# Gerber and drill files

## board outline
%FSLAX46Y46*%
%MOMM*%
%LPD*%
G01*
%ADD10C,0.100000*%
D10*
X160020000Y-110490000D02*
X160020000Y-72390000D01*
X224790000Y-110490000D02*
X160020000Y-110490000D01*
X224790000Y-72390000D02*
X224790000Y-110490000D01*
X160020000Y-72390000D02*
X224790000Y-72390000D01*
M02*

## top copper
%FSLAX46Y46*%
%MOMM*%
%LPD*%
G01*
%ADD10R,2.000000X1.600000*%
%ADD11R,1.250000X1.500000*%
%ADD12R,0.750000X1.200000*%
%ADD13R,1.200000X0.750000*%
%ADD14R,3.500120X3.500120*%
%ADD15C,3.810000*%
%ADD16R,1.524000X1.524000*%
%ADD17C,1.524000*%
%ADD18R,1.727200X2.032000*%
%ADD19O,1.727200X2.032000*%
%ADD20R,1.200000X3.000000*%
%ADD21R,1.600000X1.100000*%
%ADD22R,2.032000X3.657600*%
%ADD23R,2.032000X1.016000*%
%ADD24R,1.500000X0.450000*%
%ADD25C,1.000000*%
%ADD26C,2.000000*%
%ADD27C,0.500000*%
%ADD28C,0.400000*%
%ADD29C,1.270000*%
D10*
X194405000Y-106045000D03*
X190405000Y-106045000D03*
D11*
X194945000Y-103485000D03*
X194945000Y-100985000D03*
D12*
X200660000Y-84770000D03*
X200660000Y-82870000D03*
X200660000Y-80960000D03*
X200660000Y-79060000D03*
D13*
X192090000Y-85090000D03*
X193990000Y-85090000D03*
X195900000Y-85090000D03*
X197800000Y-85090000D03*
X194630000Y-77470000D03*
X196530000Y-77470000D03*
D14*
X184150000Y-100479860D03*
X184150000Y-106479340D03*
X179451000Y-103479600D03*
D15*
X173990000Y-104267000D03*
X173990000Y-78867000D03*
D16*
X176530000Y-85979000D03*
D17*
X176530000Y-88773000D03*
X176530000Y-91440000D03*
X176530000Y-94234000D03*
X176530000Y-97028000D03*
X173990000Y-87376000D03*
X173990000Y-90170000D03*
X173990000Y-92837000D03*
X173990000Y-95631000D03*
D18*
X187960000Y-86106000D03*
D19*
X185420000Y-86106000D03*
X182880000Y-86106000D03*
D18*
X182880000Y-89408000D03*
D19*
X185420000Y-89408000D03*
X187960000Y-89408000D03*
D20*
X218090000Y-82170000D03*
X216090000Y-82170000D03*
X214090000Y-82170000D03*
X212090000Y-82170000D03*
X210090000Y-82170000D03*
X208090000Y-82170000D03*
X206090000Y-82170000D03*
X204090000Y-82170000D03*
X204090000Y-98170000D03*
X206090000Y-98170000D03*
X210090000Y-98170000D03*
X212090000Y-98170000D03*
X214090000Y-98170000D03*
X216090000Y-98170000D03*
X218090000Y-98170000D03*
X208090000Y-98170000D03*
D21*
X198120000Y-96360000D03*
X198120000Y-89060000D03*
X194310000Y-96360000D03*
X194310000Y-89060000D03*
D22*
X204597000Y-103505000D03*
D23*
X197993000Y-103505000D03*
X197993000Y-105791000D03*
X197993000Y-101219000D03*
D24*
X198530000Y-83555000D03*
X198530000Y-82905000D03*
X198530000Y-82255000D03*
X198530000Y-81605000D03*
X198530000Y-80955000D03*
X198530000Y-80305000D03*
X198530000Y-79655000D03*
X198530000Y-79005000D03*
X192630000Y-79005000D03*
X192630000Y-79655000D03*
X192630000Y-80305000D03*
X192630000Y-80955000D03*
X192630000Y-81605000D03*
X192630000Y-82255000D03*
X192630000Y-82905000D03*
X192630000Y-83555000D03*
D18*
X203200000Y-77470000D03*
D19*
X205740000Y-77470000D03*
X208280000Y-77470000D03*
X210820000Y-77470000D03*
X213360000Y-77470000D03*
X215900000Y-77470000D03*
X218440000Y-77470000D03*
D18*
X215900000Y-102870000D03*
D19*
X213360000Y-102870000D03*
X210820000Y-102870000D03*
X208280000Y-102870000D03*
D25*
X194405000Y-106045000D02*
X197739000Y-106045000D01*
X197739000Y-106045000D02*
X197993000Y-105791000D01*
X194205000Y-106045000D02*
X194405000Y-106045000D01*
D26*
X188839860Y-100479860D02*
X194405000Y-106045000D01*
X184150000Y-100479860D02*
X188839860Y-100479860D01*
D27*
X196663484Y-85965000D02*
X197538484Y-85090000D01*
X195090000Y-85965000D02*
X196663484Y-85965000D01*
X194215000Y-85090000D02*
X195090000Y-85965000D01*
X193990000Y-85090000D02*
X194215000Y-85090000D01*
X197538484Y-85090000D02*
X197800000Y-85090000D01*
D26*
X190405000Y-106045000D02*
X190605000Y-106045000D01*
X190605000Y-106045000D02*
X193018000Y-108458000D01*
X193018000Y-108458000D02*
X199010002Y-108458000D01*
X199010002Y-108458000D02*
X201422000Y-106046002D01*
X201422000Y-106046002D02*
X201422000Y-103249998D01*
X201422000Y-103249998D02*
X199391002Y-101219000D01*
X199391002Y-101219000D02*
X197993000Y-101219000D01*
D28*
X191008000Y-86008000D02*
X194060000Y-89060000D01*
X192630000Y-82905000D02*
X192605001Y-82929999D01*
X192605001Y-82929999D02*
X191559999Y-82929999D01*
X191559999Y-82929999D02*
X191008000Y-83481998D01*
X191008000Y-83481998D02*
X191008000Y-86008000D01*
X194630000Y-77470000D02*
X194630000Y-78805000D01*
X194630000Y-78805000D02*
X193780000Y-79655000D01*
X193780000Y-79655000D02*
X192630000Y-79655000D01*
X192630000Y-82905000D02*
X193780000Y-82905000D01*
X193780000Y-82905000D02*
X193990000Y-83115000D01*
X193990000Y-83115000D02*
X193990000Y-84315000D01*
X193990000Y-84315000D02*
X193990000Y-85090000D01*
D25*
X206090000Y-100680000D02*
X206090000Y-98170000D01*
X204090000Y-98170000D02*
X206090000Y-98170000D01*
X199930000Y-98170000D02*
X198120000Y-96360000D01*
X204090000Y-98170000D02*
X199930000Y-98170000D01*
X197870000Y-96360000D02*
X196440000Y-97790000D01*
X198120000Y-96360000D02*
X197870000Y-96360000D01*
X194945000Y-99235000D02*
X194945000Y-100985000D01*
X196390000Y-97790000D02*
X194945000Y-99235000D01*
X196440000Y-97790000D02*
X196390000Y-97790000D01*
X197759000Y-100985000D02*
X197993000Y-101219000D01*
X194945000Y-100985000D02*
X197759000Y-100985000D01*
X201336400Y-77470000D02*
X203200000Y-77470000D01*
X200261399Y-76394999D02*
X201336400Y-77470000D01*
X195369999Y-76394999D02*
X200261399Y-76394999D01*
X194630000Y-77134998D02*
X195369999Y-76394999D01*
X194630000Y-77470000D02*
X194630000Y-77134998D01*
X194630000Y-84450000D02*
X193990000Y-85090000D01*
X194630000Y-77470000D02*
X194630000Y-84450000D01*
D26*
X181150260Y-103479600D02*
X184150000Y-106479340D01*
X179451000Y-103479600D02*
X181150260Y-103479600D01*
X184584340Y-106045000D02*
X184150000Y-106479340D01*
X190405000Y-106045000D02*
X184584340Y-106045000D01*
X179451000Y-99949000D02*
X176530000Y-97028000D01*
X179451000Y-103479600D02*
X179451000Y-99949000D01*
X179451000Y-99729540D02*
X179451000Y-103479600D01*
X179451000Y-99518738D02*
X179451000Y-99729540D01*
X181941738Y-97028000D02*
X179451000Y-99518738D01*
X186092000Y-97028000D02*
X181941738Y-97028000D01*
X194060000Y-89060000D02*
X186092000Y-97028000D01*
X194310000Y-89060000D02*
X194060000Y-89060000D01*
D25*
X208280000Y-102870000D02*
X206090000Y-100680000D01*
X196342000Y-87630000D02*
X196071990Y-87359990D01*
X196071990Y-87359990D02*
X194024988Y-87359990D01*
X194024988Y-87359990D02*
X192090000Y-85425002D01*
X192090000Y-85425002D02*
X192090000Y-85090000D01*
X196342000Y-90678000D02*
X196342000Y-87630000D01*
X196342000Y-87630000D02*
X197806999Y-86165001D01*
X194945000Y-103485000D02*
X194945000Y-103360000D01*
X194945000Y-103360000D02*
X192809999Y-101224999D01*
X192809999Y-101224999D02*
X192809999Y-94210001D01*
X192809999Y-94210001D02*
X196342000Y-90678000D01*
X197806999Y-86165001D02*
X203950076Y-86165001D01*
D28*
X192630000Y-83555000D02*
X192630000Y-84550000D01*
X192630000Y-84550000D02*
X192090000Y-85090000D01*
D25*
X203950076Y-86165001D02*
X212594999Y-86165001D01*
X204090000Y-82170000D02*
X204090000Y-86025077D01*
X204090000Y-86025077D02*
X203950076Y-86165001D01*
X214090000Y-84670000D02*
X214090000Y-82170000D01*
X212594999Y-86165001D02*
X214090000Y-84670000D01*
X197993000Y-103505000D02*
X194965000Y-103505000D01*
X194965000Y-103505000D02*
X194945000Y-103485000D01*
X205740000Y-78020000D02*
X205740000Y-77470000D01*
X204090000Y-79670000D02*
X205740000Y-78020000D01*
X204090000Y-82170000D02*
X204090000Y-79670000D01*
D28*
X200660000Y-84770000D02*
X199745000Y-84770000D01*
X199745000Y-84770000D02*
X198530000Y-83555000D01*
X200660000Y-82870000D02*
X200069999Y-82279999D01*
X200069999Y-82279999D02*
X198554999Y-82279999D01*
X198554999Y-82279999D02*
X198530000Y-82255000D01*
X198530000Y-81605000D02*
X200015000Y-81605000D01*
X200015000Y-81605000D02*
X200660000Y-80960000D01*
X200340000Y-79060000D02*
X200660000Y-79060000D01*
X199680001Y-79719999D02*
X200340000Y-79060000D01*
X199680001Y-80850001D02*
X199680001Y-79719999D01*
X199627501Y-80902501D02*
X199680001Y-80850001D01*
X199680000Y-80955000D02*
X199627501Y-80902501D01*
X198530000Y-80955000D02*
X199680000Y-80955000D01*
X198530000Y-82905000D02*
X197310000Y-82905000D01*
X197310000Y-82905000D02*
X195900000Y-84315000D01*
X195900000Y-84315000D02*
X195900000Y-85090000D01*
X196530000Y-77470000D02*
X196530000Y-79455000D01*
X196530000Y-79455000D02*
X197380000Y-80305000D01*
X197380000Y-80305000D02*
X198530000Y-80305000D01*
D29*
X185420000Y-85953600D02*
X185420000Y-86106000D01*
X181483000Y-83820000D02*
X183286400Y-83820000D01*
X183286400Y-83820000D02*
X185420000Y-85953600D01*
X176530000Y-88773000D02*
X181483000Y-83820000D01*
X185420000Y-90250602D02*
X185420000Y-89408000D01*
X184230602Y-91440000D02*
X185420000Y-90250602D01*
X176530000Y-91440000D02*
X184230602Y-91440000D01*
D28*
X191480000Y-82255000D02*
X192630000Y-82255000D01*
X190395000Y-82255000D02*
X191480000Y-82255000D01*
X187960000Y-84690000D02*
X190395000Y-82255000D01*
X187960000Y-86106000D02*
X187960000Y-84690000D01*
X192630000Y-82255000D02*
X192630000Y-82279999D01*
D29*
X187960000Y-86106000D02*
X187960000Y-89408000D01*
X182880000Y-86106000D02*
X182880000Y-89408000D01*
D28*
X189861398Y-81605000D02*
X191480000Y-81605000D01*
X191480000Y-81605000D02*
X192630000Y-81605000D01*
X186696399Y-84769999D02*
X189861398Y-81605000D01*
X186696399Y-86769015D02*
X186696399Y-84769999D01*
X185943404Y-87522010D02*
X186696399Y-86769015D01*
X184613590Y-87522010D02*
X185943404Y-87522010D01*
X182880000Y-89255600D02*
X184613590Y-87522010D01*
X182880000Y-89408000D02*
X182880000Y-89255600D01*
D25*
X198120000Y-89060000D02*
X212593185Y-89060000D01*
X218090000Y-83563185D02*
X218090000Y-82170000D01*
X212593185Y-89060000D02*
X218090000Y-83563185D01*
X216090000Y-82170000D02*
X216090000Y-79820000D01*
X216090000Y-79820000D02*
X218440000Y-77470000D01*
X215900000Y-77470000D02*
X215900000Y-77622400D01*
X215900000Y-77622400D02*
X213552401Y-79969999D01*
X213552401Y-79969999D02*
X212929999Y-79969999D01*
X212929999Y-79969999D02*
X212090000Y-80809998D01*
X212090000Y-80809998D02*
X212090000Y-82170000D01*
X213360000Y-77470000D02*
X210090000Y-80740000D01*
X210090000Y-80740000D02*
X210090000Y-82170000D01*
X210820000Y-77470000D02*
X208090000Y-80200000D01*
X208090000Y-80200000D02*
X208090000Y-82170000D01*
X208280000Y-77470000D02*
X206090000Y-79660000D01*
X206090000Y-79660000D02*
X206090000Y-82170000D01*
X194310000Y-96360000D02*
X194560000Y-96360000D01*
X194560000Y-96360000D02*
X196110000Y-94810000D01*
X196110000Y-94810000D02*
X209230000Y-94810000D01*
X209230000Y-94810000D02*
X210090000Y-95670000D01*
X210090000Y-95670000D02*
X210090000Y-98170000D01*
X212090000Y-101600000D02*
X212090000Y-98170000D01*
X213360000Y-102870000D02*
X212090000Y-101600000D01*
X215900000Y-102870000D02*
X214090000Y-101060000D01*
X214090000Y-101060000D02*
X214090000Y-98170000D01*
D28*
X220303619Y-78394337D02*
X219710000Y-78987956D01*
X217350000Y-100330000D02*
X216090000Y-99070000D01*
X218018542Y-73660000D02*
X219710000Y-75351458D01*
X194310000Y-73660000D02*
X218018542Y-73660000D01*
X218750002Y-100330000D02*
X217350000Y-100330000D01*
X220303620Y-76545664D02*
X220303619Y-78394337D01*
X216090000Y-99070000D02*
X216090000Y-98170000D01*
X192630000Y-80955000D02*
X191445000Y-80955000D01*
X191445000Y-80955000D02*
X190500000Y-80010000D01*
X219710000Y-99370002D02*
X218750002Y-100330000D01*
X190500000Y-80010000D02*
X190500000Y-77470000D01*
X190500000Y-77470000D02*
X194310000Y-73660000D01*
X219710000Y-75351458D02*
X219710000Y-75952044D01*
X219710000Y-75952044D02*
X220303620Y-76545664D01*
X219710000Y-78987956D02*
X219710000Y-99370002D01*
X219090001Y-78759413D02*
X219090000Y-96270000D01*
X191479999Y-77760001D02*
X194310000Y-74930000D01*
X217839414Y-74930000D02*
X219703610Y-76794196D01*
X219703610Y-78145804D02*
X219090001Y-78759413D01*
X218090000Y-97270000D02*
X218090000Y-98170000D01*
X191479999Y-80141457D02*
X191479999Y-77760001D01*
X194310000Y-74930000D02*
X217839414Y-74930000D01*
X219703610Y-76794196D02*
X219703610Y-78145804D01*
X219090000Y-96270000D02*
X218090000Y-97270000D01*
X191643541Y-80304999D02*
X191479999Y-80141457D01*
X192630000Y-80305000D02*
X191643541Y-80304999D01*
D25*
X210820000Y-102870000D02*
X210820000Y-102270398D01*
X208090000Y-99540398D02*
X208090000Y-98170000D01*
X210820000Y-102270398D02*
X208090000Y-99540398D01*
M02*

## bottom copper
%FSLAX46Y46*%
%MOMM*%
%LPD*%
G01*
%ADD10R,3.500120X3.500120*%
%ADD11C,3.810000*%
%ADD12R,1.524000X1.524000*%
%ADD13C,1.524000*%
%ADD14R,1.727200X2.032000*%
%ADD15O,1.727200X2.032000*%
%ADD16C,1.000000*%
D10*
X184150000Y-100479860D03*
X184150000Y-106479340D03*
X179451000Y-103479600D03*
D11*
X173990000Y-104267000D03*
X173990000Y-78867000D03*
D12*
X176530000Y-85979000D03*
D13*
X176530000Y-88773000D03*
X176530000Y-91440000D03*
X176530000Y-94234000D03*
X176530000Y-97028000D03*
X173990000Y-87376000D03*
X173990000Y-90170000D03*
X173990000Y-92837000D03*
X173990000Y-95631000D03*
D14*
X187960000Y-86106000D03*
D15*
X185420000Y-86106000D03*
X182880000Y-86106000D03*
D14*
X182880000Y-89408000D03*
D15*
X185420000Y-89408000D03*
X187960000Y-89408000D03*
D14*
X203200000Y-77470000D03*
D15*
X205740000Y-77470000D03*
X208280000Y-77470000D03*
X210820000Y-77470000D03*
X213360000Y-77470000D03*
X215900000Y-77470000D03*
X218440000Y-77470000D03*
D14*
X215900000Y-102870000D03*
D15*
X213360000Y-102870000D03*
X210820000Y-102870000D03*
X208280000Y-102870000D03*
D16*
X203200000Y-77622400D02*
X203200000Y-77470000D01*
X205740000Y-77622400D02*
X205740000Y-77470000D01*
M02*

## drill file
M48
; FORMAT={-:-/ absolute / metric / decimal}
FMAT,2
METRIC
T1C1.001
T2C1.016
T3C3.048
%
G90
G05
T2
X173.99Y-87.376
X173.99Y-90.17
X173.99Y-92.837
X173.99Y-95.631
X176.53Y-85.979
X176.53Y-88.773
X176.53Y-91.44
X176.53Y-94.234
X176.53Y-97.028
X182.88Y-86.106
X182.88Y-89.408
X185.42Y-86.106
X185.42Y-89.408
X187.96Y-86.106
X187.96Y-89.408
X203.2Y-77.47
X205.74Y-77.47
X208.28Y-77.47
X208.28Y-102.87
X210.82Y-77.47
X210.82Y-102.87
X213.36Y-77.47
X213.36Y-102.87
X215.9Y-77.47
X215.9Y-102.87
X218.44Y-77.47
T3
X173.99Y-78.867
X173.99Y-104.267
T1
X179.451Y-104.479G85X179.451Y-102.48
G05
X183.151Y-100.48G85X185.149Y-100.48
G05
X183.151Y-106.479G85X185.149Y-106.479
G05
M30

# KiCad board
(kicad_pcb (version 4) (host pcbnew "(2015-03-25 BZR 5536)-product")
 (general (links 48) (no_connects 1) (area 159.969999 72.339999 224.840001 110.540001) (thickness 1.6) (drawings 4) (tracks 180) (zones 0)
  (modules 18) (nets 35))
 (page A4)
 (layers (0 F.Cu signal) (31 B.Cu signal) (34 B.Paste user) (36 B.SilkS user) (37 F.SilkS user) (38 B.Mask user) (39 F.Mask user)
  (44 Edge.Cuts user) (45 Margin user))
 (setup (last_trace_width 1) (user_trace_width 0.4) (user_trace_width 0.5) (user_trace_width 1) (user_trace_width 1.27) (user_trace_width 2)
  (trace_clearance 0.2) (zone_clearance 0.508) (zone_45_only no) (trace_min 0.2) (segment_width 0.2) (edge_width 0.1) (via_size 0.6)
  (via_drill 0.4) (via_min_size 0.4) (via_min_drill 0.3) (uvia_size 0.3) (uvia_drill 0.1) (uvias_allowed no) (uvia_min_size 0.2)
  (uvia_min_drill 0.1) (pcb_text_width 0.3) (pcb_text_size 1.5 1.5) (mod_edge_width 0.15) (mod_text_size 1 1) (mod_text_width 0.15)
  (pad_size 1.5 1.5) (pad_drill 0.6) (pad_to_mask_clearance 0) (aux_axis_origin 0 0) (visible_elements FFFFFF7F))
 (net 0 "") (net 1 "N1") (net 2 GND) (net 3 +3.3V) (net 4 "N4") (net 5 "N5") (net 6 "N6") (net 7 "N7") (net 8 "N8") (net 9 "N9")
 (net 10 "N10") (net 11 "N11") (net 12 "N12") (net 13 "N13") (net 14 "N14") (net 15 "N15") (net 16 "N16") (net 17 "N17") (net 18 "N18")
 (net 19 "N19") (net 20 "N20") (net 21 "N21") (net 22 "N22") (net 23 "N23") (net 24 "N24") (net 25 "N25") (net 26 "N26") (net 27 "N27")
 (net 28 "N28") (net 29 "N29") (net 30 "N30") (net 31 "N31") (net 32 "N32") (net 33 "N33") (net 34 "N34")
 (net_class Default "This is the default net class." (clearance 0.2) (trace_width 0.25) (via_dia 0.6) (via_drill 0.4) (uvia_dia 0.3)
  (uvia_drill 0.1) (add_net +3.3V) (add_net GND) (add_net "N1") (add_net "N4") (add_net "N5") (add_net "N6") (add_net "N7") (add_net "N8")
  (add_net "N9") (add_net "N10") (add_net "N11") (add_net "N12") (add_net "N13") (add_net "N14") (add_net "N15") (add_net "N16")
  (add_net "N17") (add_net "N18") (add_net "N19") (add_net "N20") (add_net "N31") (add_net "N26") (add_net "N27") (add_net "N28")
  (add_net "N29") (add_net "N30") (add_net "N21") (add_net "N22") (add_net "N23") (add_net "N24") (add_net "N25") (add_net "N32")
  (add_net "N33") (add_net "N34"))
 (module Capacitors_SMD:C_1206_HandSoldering (layer F.Cu) (at 192.405 106.045 180)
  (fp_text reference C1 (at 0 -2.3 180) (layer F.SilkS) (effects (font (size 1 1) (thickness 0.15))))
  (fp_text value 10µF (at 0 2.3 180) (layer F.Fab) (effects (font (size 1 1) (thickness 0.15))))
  (pad 1 smd rect (at -2 0 180) (size 2 1.6) (layers F.Cu F.Mask) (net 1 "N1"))
  (pad 2 smd rect (at 2 0 180) (size 2 1.6) (layers F.Cu F.Mask) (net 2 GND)))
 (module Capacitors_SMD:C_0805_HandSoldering (layer F.Cu) (at 194.945 102.235 90)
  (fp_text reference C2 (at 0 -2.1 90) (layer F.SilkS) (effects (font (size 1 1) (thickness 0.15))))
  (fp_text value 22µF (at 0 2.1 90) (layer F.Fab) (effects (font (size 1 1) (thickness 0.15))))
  (pad 1 smd rect (at -1.25 0 90) (size 1.5 1.25) (layers F.Cu F.Mask) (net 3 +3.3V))
  (pad 2 smd rect (at 1.25 0 90) (size 1.5 1.25) (layers F.Cu F.Mask) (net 2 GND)))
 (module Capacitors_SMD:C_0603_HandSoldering (layer F.Cu) (at 200.66 83.82 90)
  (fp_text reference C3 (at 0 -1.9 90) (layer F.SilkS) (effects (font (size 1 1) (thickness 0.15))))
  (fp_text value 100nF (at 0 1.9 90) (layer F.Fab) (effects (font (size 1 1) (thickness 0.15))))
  (pad 1 smd rect (at -0.95 0 90) (size 1.2 0.75) (layers F.Cu F.Mask) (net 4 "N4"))
  (pad 2 smd rect (at 0.95 0 90) (size 1.2 0.75) (layers F.Cu F.Mask) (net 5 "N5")))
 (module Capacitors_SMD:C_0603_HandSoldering (layer F.Cu) (at 200.66 80.01 90)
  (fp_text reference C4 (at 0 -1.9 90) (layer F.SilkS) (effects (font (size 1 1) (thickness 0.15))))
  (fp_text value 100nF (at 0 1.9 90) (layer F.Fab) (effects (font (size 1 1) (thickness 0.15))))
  (pad 1 smd rect (at -0.95 0 90) (size 1.2 0.75) (layers F.Cu F.Mask) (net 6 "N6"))
  (pad 2 smd rect (at 0.95 0 90) (size 1.2 0.75) (layers F.Cu F.Mask) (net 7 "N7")))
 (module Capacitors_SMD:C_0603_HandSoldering (layer F.Cu) (at 193.04 85.09)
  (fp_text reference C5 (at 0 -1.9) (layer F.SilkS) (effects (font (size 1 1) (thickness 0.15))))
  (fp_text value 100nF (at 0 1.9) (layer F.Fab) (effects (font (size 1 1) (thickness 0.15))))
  (pad 1 smd rect (at -0.95 0) (size 1.2 0.75) (layers F.Cu F.Mask) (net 3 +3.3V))
  (pad 2 smd rect (at 0.95 0) (size 1.2 0.75) (layers F.Cu F.Mask) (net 2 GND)))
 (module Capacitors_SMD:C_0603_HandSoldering (layer F.Cu) (at 196.85 85.09)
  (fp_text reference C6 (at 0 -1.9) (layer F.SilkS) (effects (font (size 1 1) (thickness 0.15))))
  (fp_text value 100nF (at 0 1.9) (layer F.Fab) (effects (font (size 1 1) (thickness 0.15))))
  (pad 1 smd rect (at -0.95 0) (size 1.2 0.75) (layers F.Cu F.Mask) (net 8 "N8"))
  (pad 2 smd rect (at 0.95 0) (size 1.2 0.75) (layers F.Cu F.Mask) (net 2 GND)))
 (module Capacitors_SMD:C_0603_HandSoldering (layer F.Cu) (at 195.58 77.47)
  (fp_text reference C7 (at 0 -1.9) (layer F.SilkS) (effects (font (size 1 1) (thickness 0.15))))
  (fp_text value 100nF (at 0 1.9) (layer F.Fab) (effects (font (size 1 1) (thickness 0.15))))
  (pad 1 smd rect (at -0.95 0) (size 1.2 0.75) (layers F.Cu F.Mask) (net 2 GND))
  (pad 2 smd rect (at 0.95 0) (size 1.2 0.75) (layers F.Cu F.Mask) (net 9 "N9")))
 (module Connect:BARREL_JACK (layer B.Cu) (at 184.15 106.68 90)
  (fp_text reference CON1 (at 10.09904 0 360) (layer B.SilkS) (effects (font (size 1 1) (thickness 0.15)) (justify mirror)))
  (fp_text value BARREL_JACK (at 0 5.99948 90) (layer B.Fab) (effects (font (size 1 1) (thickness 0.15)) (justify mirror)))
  (pad 1 thru_hole rect (at 6.20014 0 90) (size 3.50012 3.50012) (drill oval 1.00076 2.99974) (layers *.Cu *.Mask B.SilkS) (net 1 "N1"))
  (pad 2 thru_hole rect (at 0.20066 0 90) (size 3.50012 3.50012) (drill oval 1.00076 2.99974) (layers *.Cu *.Mask B.SilkS) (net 2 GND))
  (pad 3 thru_hole rect (at 3.2004 -4.699 90) (size 3.50012 3.50012) (drill oval 2.99974 1.00076) (layers *.Cu *.Mask B.SilkS) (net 2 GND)))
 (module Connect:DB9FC (layer B.Cu) (at 175.26 91.44 270)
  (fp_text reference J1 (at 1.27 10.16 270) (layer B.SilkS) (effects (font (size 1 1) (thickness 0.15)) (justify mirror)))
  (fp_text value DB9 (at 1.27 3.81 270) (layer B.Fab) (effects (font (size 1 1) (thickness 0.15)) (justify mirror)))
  (pad "" thru_hole circle (at 12.827 1.27 270) (size 3.81 3.81) (drill 3.048) (layers *.Cu *.Mask B.SilkS))
  (pad "" thru_hole circle (at -12.573 1.27 270) (size 3.81 3.81) (drill 3.048) (layers *.Cu *.Mask B.SilkS))
  (pad 1 thru_hole rect (at -5.461 -1.27 270) (size 1.524 1.524) (drill 1.016) (layers *.Cu *.Mask B.SilkS) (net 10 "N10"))
  (pad 2 thru_hole circle (at -2.667 -1.27 270) (size 1.524 1.524) (drill 1.016) (layers *.Cu *.Mask B.SilkS) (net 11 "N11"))
  (pad 3 thru_hole circle (at 0 -1.27 270) (size 1.524 1.524) (drill 1.016) (layers *.Cu *.Mask B.SilkS) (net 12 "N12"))
  (pad 4 thru_hole circle (at 2.794 -1.27 270) (size 1.524 1.524) (drill 1.016) (layers *.Cu *.Mask B.SilkS) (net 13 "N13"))
  (pad 5 thru_hole circle (at 5.588 -1.27 270) (size 1.524 1.524) (drill 1.016) (layers *.Cu *.Mask B.SilkS) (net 2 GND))
  (pad 6 thru_hole circle (at -4.064 1.27 270) (size 1.524 1.524) (drill 1.016) (layers *.Cu *.Mask B.SilkS) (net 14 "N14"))
  (pad 7 thru_hole circle (at -1.27 1.27 270) (size 1.524 1.524) (drill 1.016) (layers *.Cu *.Mask B.SilkS) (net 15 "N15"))
  (pad 8 thru_hole circle (at 1.397 1.27 270) (size 1.524 1.524) (drill 1.016) (layers *.Cu *.Mask B.SilkS) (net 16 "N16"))
  (pad 9 thru_hole circle (at 4.191 1.27 270) (size 1.524 1.524) (drill 1.016) (layers *.Cu *.Mask B.SilkS) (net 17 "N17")))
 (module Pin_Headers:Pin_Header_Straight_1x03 (layer B.Cu) (at 187.96 86.106 90)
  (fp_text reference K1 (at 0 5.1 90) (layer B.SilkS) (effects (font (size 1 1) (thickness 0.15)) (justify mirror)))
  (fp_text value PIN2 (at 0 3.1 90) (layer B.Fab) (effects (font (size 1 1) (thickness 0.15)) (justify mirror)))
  (pad 1 thru_hole rect (at 0 0 90) (size 2.032 1.7272) (drill 1.016) (layers *.Cu *.Mask B.SilkS) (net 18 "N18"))
  (pad 2 thru_hole oval (at 0 -2.54 90) (size 2.032 1.7272) (drill 1.016) (layers *.Cu *.Mask B.SilkS) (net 11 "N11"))
  (pad 3 thru_hole oval (at 0 -5.08 90) (size 2.032 1.7272) (drill 1.016) (layers *.Cu *.Mask B.SilkS) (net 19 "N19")))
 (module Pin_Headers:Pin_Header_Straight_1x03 (layer B.Cu) (at 182.88 89.408 270)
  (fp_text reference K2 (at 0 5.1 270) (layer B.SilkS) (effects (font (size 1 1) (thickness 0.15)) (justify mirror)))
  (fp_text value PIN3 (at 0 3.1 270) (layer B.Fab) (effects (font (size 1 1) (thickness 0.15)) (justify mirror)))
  (pad 1 thru_hole rect (at 0 0 270) (size 2.032 1.7272) (drill 1.016) (layers *.Cu *.Mask B.SilkS) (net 19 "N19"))
  (pad 2 thru_hole oval (at 0 -2.54 270) (size 2.032 1.7272) (drill 1.016) (layers *.Cu *.Mask B.SilkS) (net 12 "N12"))
  (pad 3 thru_hole oval (at 0 -5.08 270) (size 2.032 1.7272) (drill 1.016) (layers *.Cu *.Mask B.SilkS) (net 18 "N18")))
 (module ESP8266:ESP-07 (layer F.Cu) (at 212.09 90.17 180)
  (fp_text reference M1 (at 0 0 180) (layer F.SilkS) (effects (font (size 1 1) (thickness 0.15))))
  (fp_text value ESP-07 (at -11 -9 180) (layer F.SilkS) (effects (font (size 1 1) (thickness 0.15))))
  (pad 1 smd rect (at -6 8 180) (size 1.2 3) (layers F.Cu F.Mask) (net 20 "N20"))
  (pad 2 smd rect (at -4 8 180) (size 1.2 3) (layers F.Cu F.Mask) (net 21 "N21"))
  (pad 3 smd rect (at -2 8 180) (size 1.2 3) (layers F.Cu F.Mask) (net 3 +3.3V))
  (pad 4 smd rect (at 0 8 180) (size 1.2 3) (layers F.Cu F.Mask) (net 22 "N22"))
  (pad 5 smd rect (at 2 8 180) (size 1.2 3) (layers F.Cu F.Mask) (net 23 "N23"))
  (pad 6 smd rect (at 4 8 180) (size 1.2 3) (layers F.Cu F.Mask) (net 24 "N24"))
  (pad 7 smd rect (at 6 8 180) (size 1.2 3) (layers F.Cu F.Mask) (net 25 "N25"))
  (pad 8 smd rect (at 8 8 180) (size 1.2 3) (layers F.Cu F.Mask) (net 3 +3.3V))
  (pad 9 smd rect (at 8 -8 180) (size 1.2 3) (layers F.Cu F.Mask) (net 2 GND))
  (pad 10 smd rect (at 6 -8 180) (size 1.2 3) (layers F.Cu F.Mask) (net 2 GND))
  (pad 12 smd rect (at 2 -8 180) (size 1.2 3) (layers F.Cu F.Mask) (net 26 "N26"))
  (pad 13 smd rect (at 0 -8 180) (size 1.2 3) (layers F.Cu F.Mask) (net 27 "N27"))
  (pad 14 smd rect (at -2 -8 180) (size 1.2 3) (layers F.Cu F.Mask) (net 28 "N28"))
  (pad 15 smd rect (at -4 -8 180) (size 1.2 3) (layers F.Cu F.Mask) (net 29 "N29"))
  (pad 16 smd rect (at -6 -8 180) (size 1.2 3) (layers F.Cu F.Mask) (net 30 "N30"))
  (pad 11 smd rect (at 4 -8 180) (size 1.2 3) (layers F.Cu F.Mask) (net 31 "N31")))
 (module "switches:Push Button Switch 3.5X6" (layer F.Cu) (at 198.12 92.71 90)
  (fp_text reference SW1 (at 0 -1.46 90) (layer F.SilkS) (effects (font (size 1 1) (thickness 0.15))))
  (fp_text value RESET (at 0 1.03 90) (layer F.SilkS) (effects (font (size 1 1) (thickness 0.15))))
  (pad 1 smd rect (at -3.65 0 90) (size 1.1 1.6) (layers F.Cu F.Mask) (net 2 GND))
  (pad 2 smd rect (at 3.65 0 90) (size 1.1 1.6) (layers F.Cu F.Mask) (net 20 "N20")))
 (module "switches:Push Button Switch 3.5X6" (layer F.Cu) (at 194.31 92.71 90)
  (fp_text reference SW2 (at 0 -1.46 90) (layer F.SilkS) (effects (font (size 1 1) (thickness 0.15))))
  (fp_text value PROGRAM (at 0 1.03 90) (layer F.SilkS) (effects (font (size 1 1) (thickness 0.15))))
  (pad 1 smd rect (at -3.65 0 90) (size 1.1 1.6) (layers F.Cu F.Mask) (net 26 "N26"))
  (pad 2 smd rect (at 3.65 0 90) (size 1.1 1.6) (layers F.Cu F.Mask) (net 2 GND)))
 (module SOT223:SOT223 (layer F.Cu) (at 201.295 103.505 270)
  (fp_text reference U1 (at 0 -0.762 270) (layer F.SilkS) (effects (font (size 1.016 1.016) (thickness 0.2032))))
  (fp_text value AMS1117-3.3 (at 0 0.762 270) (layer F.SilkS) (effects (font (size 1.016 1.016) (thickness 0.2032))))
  (pad 4 smd rect (at 0 -3.302 270) (size 3.6576 2.032) (layers F.Cu F.Mask))
  (pad 2 smd rect (at 0 3.302 270) (size 1.016 2.032) (layers F.Cu F.Mask) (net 3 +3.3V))
  (pad 3 smd rect (at 2.286 3.302 270) (size 1.016 2.032) (layers F.Cu F.Mask) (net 1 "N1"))
  (pad 1 smd rect (at -2.286 3.302 270) (size 1.016 2.032) (layers F.Cu F.Mask) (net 2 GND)))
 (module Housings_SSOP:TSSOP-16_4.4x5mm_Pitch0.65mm (layer F.Cu) (at 195.58 81.28 180)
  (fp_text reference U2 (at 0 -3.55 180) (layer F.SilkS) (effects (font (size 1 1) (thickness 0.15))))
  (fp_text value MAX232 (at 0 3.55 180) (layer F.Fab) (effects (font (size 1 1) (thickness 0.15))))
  (pad 1 smd rect (at -2.95 -2.275 180) (size 1.5 0.45) (layers F.Cu F.Mask) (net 4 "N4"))
  (pad 2 smd rect (at -2.95 -1.625 180) (size 1.5 0.45) (layers F.Cu F.Mask) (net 8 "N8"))
  (pad 3 smd rect (at -2.95 -0.975 180) (size 1.5 0.45) (layers F.Cu F.Mask) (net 5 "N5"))
  (pad 4 smd rect (at -2.95 -0.325 180) (size 1.5 0.45) (layers F.Cu F.Mask) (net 6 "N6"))
  (pad 5 smd rect (at -2.95 0.325 180) (size 1.5 0.45) (layers F.Cu F.Mask) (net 7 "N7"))
  (pad 6 smd rect (at -2.95 0.975 180) (size 1.5 0.45) (layers F.Cu F.Mask) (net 9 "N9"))
  (pad 7 smd rect (at -2.95 1.625 180) (size 1.5 0.45) (layers F.Cu F.Mask) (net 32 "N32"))
  (pad 8 smd rect (at -2.95 2.275 180) (size 1.5 0.45) (layers F.Cu F.Mask) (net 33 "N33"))
  (pad 9 smd rect (at 2.95 2.275 180) (size 1.5 0.45) (layers F.Cu F.Mask) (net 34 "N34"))
  (pad 10 smd rect (at 2.95 1.625 180) (size 1.5 0.45) (layers F.Cu F.Mask) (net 2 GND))
  (pad 11 smd rect (at 2.95 0.975 180) (size 1.5 0.45) (layers F.Cu F.Mask) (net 30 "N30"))
  (pad 12 smd rect (at 2.95 0.325 180) (size 1.5 0.45) (layers F.Cu F.Mask) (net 29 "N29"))
  (pad 13 smd rect (at 2.95 -0.325 180) (size 1.5 0.45) (layers F.Cu F.Mask) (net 19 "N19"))
  (pad 14 smd rect (at 2.95 -0.975 180) (size 1.5 0.45) (layers F.Cu F.Mask) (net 18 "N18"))
  (pad 15 smd rect (at 2.95 -1.625 180) (size 1.5 0.45) (layers F.Cu F.Mask) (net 2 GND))
  (pad 16 smd rect (at 2.95 -2.275 180) (size 1.5 0.45) (layers F.Cu F.Mask) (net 3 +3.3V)))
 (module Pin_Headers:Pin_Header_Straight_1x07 (layer F.Cu) (at 203.2 77.47 90)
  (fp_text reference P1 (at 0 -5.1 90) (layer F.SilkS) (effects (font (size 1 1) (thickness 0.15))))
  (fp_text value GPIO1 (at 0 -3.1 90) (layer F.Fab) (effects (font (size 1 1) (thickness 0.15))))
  (pad 1 thru_hole rect (at 0 0 90) (size 2.032 1.7272) (drill 1.016) (layers *.Cu *.Mask F.SilkS) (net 2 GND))
  (pad 2 thru_hole oval (at 0 2.54 90) (size 2.032 1.7272) (drill 1.016) (layers *.Cu *.Mask F.SilkS) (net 3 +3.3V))
  (pad 3 thru_hole oval (at 0 5.08 90) (size 2.032 1.7272) (drill 1.016) (layers *.Cu *.Mask F.SilkS) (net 25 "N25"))
  (pad 4 thru_hole oval (at 0 7.62 90) (size 2.032 1.7272) (drill 1.016) (layers *.Cu *.Mask F.SilkS) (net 24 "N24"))
  (pad 5 thru_hole oval (at 0 10.16 90) (size 2.032 1.7272) (drill 1.016) (layers *.Cu *.Mask F.SilkS) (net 23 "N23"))
  (pad 6 thru_hole oval (at 0 12.7 90) (size 2.032 1.7272) (drill 1.016) (layers *.Cu *.Mask F.SilkS) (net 22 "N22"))
  (pad 7 thru_hole oval (at 0 15.24 90) (size 2.032 1.7272) (drill 1.016) (layers *.Cu *.Mask F.SilkS) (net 21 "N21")))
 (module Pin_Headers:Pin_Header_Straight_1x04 (layer F.Cu) (at 215.9 102.87 270)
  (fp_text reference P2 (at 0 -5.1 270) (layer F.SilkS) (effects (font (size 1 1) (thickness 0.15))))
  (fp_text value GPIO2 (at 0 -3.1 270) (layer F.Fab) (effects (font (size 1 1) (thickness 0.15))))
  (pad 1 thru_hole rect (at 0 0 270) (size 2.032 1.7272) (drill 1.016) (layers *.Cu *.Mask F.SilkS) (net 28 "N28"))
  (pad 2 thru_hole oval (at 0 2.54 270) (size 2.032 1.7272) (drill 1.016) (layers *.Cu *.Mask F.SilkS) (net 27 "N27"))
  (pad 3 thru_hole oval (at 0 5.08 270) (size 2.032 1.7272) (drill 1.016) (layers *.Cu *.Mask F.SilkS) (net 31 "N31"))
  (pad 4 thru_hole oval (at 0 7.62 270) (size 2.032 1.7272) (drill 1.016) (layers *.Cu *.Mask F.SilkS) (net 2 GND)))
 (gr_line (start 160.02 110.49) (end 160.02 72.39) (angle 90) (layer Edge.Cuts) (width 0.1))
 (gr_line (start 224.79 110.49) (end 160.02 110.49) (angle 90) (layer Edge.Cuts) (width 0.1))
 (gr_line (start 224.79 72.39) (end 224.79 110.49) (angle 90) (layer Edge.Cuts) (width 0.1))
 (gr_line (start 160.02 72.39) (end 224.79 72.39) (angle 90) (layer Edge.Cuts) (width 0.1))
 (segment (start 194.405 106.045) (end 197.739 106.045) (width 1) (layer F.Cu) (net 1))
 (segment (start 197.739 106.045) (end 197.993 105.791) (width 1) (layer F.Cu) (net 1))
 (segment (start 194.205 106.045) (end 194.405 106.045) (width 1) (layer F.Cu) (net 1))
 (segment (start 188.83986 100.47986) (end 194.405 106.045) (width 2) (layer F.Cu) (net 1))
 (segment (start 184.15 100.47986) (end 188.83986 100.47986) (width 2) (layer F.Cu) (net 1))
 (segment (start 196.663484 85.965) (end 197.538484 85.09) (width 0.5) (layer F.Cu) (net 2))
 (segment (start 195.09 85.965) (end 196.663484 85.965) (width 0.5) (layer F.Cu) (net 2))
 (segment (start 194.215 85.09) (end 195.09 85.965) (width 0.5) (layer F.Cu) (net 2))
 (segment (start 193.99 85.09) (end 194.215 85.09) (width 0.5) (layer F.Cu) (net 2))
 (segment (start 197.538484 85.09) (end 197.8 85.09) (width 0.5) (layer F.Cu) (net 2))
 (segment (start 190.405 106.045) (end 190.605 106.045) (width 2) (layer F.Cu) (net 2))
 (segment (start 190.605 106.045) (end 193.018 108.458) (width 2) (layer F.Cu) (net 2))
 (segment (start 193.018 108.458) (end 199.010002 108.458) (width 2) (layer F.Cu) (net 2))
 (segment (start 199.010002 108.458) (end 201.422 106.046002) (width 2) (layer F.Cu) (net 2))
 (segment (start 201.422 106.046002) (end 201.422 103.249998) (width 2) (layer F.Cu) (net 2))
 (segment (start 201.422 103.249998) (end 199.391002 101.219) (width 2) (layer F.Cu) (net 2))
 (segment (start 199.391002 101.219) (end 197.993 101.219) (width 2) (layer F.Cu) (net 2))
 (segment (start 191.008 86.008) (end 194.06 89.06) (width 0.4) (layer F.Cu) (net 2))
 (segment (start 192.63 82.905) (end 192.605001 82.929999) (width 0.4) (layer F.Cu) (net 2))
 (segment (start 192.605001 82.929999) (end 191.559999 82.929999) (width 0.4) (layer F.Cu) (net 2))
 (segment (start 191.559999 82.929999) (end 191.008 83.481998) (width 0.4) (layer F.Cu) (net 2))
 (segment (start 191.008 83.481998) (end 191.008 86.008) (width 0.4) (layer F.Cu) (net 2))
 (segment (start 194.63 77.47) (end 194.63 78.805) (width 0.4) (layer F.Cu) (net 2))
 (segment (start 194.63 78.805) (end 193.78 79.655) (width 0.4) (layer F.Cu) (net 2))
 (segment (start 193.78 79.655) (end 192.63 79.655) (width 0.4) (layer F.Cu) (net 2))
 (segment (start 192.63 82.905) (end 193.78 82.905) (width 0.4) (layer F.Cu) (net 2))
 (segment (start 193.78 82.905) (end 193.99 83.115) (width 0.4) (layer F.Cu) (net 2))
 (segment (start 193.99 83.115) (end 193.99 84.315) (width 0.4) (layer F.Cu) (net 2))
 (segment (start 193.99 84.315) (end 193.99 85.09) (width 0.4) (layer F.Cu) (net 2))
 (segment (start 206.09 100.68) (end 206.09 98.17) (width 1) (layer F.Cu) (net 2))
 (segment (start 204.09 98.17) (end 206.09 98.17) (width 1) (layer F.Cu) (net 2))
 (segment (start 199.93 98.17) (end 198.12 96.36) (width 1) (layer F.Cu) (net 2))
 (segment (start 204.09 98.17) (end 199.93 98.17) (width 1) (layer F.Cu) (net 2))
 (segment (start 197.87 96.36) (end 196.44 97.79) (width 1) (layer F.Cu) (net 2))
 (segment (start 198.12 96.36) (end 197.87 96.36) (width 1) (layer F.Cu) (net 2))
 (segment (start 194.945 99.235) (end 194.945 100.985) (width 1) (layer F.Cu) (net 2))
 (segment (start 196.39 97.79) (end 194.945 99.235) (width 1) (layer F.Cu) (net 2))
 (segment (start 196.44 97.79) (end 196.39 97.79) (width 1) (layer F.Cu) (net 2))
 (segment (start 197.759 100.985) (end 197.993 101.219) (width 1) (layer F.Cu) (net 2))
 (segment (start 194.945 100.985) (end 197.759 100.985) (width 1) (layer F.Cu) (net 2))
 (segment (start 201.3364 77.47) (end 203.2 77.47) (width 1) (layer F.Cu) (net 2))
 (segment (start 200.261399 76.394999) (end 201.3364 77.47) (width 1) (layer F.Cu) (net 2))
 (segment (start 195.369999 76.394999) (end 200.261399 76.394999) (width 1) (layer F.Cu) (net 2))
 (segment (start 194.63 77.134998) (end 195.369999 76.394999) (width 1) (layer F.Cu) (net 2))
 (segment (start 194.63 77.47) (end 194.63 77.134998) (width 1) (layer F.Cu) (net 2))
 (segment (start 194.63 84.45) (end 193.99 85.09) (width 1) (layer F.Cu) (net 2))
 (segment (start 194.63 77.47) (end 194.63 84.45) (width 1) (layer F.Cu) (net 2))
 (segment (start 203.2 77.6224) (end 203.2 77.47) (width 1) (layer B.Cu) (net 2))
 (segment (start 181.15026 103.4796) (end 184.15 106.47934) (width 2) (layer F.Cu) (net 2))
 (segment (start 179.451 103.4796) (end 181.15026 103.4796) (width 2) (layer F.Cu) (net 2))
 (segment (start 184.58434 106.045) (end 184.15 106.47934) (width 2) (layer F.Cu) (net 2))
 (segment (start 190.405 106.045) (end 184.58434 106.045) (width 2) (layer F.Cu) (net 2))
 (segment (start 179.451 99.949) (end 176.53 97.028) (width 2) (layer F.Cu) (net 2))
 (segment (start 179.451 103.4796) (end 179.451 99.949) (width 2) (layer F.Cu) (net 2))
 (segment (start 179.451 99.72954) (end 179.451 103.4796) (width 2) (layer F.Cu) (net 2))
 (segment (start 179.451 99.518738) (end 179.451 99.72954) (width 2) (layer F.Cu) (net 2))
 (segment (start 181.941738 97.028) (end 179.451 99.518738) (width 2) (layer F.Cu) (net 2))
 (segment (start 186.092 97.028) (end 181.941738 97.028) (width 2) (layer F.Cu) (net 2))
 (segment (start 194.06 89.06) (end 186.092 97.028) (width 2) (layer F.Cu) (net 2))
 (segment (start 194.31 89.06) (end 194.06 89.06) (width 2) (layer F.Cu) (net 2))
 (segment (start 208.28 102.87) (end 206.09 100.68) (width 1) (layer F.Cu) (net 2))
 (segment (start 196.342 87.63) (end 196.07199 87.35999) (width 1) (layer F.Cu) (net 3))
 (segment (start 196.07199 87.35999) (end 194.024988 87.35999) (width 1) (layer F.Cu) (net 3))
 (segment (start 194.024988 87.35999) (end 192.09 85.425002) (width 1) (layer F.Cu) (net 3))
 (segment (start 192.09 85.425002) (end 192.09 85.09) (width 1) (layer F.Cu) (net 3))
 (segment (start 196.342 90.678) (end 196.342 87.63) (width 1) (layer F.Cu) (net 3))
 (segment (start 196.342 87.63) (end 197.806999 86.165001) (width 1) (layer F.Cu) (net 3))
 (segment (start 194.945 103.485) (end 194.945 103.36) (width 1) (layer F.Cu) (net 3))
 (segment (start 194.945 103.36) (end 192.809999 101.224999) (width 1) (layer F.Cu) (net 3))
 (segment (start 192.809999 101.224999) (end 192.809999 94.210001) (width 1) (layer F.Cu) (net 3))
 (segment (start 192.809999 94.210001) (end 196.342 90.678) (width 1) (layer F.Cu) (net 3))
 (segment (start 197.806999 86.165001) (end 203.950076 86.165001) (width 1) (layer F.Cu) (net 3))
 (segment (start 192.63 83.555) (end 192.63 84.55) (width 0.4) (layer F.Cu) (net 3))
 (segment (start 192.63 84.55) (end 192.09 85.09) (width 0.4) (layer F.Cu) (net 3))
 (segment (start 203.950076 86.165001) (end 212.594999 86.165001) (width 1) (layer F.Cu) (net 3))
 (segment (start 204.09 82.17) (end 204.09 86.025077) (width 1) (layer F.Cu) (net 3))
 (segment (start 204.09 86.025077) (end 203.950076 86.165001) (width 1) (layer F.Cu) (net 3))
 (segment (start 214.09 84.67) (end 214.09 82.17) (width 1) (layer F.Cu) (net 3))
 (segment (start 212.594999 86.165001) (end 214.09 84.67) (width 1) (layer F.Cu) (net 3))
 (segment (start 197.993 103.505) (end 194.965 103.505) (width 1) (layer F.Cu) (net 3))
 (segment (start 194.965 103.505) (end 194.945 103.485) (width 1) (layer F.Cu) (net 3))
 (segment (start 205.74 78.02) (end 205.74 77.47) (width 1) (layer F.Cu) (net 3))
 (segment (start 204.09 79.67) (end 205.74 78.02) (width 1) (layer F.Cu) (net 3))
 (segment (start 204.09 82.17) (end 204.09 79.67) (width 1) (layer F.Cu) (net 3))
 (segment (start 205.74 77.6224) (end 205.74 77.47) (width 1) (layer B.Cu) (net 3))
 (segment (start 200.66 84.77) (end 199.745 84.77) (width 0.4) (layer F.Cu) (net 4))
 (segment (start 199.745 84.77) (end 198.53 83.555) (width 0.4) (layer F.Cu) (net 4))
 (segment (start 200.66 82.87) (end 200.069999 82.279999) (width 0.4) (layer F.Cu) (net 5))
 (segment (start 200.069999 82.279999) (end 198.554999 82.279999) (width 0.4) (layer F.Cu) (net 5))
 (segment (start 198.554999 82.279999) (end 198.53 82.255) (width 0.4) (layer F.Cu) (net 5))
 (segment (start 198.53 81.605) (end 200.015 81.605) (width 0.4) (layer F.Cu) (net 6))
 (segment (start 200.015 81.605) (end 200.66 80.96) (width 0.4) (layer F.Cu) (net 6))
 (segment (start 200.34 79.06) (end 200.66 79.06) (width 0.4) (layer F.Cu) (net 7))
 (segment (start 199.680001 79.719999) (end 200.34 79.06) (width 0.4) (layer F.Cu) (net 7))
 (segment (start 199.680001 80.850001) (end 199.680001 79.719999) (width 0.4) (layer F.Cu) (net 7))
 (segment (start 199.627501 80.902501) (end 199.680001 80.850001) (width 0.4) (layer F.Cu) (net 7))
 (segment (start 199.68 80.955) (end 199.627501 80.902501) (width 0.4) (layer F.Cu) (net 7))
 (segment (start 198.53 80.955) (end 199.68 80.955) (width 0.4) (layer F.Cu) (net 7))
 (segment (start 198.53 82.905) (end 197.31 82.905) (width 0.4) (layer F.Cu) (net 8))
 (segment (start 197.31 82.905) (end 195.9 84.315) (width 0.4) (layer F.Cu) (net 8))
 (segment (start 195.9 84.315) (end 195.9 85.09) (width 0.4) (layer F.Cu) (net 8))
 (segment (start 196.53 77.47) (end 196.53 79.455) (width 0.4) (layer F.Cu) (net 9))
 (segment (start 196.53 79.455) (end 197.38 80.305) (width 0.4) (layer F.Cu) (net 9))
 (segment (start 197.38 80.305) (end 198.53 80.305) (width 0.4) (layer F.Cu) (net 9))
 (segment (start 185.42 85.9536) (end 185.42 86.106) (width 1.27) (layer F.Cu) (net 11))
 (segment (start 181.483 83.82) (end 183.2864 83.82) (width 1.27) (layer F.Cu) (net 11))
 (segment (start 183.2864 83.82) (end 185.42 85.9536) (width 1.27) (layer F.Cu) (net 11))
 (segment (start 176.53 88.773) (end 181.483 83.82) (width 1.27) (layer F.Cu) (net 11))
 (segment (start 185.42 90.250602) (end 185.42 89.408) (width 1.27) (layer F.Cu) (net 12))
 (segment (start 184.230602 91.44) (end 185.42 90.250602) (width 1.27) (layer F.Cu) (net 12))
 (segment (start 176.53 91.44) (end 184.230602 91.44) (width 1.27) (layer F.Cu) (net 12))
 (segment (start 191.48 82.255) (end 192.63 82.255) (width 0.4) (layer F.Cu) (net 18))
 (segment (start 190.395 82.255) (end 191.48 82.255) (width 0.4) (layer F.Cu) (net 18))
 (segment (start 187.96 84.69) (end 190.395 82.255) (width 0.4) (layer F.Cu) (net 18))
 (segment (start 187.96 86.106) (end 187.96 84.69) (width 0.4) (layer F.Cu) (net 18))
 (segment (start 192.63 82.255) (end 192.63 82.279999) (width 0.4) (layer F.Cu) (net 18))
 (segment (start 187.96 86.106) (end 187.96 89.408) (width 1.27) (layer F.Cu) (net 18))
 (segment (start 182.88 86.106) (end 182.88 89.408) (width 1.27) (layer F.Cu) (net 19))
 (segment (start 189.861398 81.605) (end 191.48 81.605) (width 0.4) (layer F.Cu) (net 19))
 (segment (start 191.48 81.605) (end 192.63 81.605) (width 0.4) (layer F.Cu) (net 19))
 (segment (start 186.696399 84.769999) (end 189.861398 81.605) (width 0.4) (layer F.Cu) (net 19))
 (segment (start 186.696399 86.769015) (end 186.696399 84.769999) (width 0.4) (layer F.Cu) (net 19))
 (segment (start 185.943404 87.52201) (end 186.696399 86.769015) (width 0.4) (layer F.Cu) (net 19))
 (segment (start 184.61359 87.52201) (end 185.943404 87.52201) (width 0.4) (layer F.Cu) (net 19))
 (segment (start 182.88 89.2556) (end 184.61359 87.52201) (width 0.4) (layer F.Cu) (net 19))
 (segment (start 182.88 89.408) (end 182.88 89.2556) (width 0.4) (layer F.Cu) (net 19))
 (segment (start 198.12 89.06) (end 212.593185 89.06) (width 1) (layer F.Cu) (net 20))
 (segment (start 218.09 83.563185) (end 218.09 82.17) (width 1) (layer F.Cu) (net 20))
 (segment (start 212.593185 89.06) (end 218.09 83.563185) (width 1) (layer F.Cu) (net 20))
 (segment (start 216.09 82.17) (end 216.09 79.82) (width 1) (layer F.Cu) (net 21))
 (segment (start 216.09 79.82) (end 218.44 77.47) (width 1) (layer F.Cu) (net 21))
 (segment (start 215.9 77.47) (end 215.9 77.6224) (width 1) (layer F.Cu) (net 22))
 (segment (start 215.9 77.6224) (end 213.552401 79.969999) (width 1) (layer F.Cu) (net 22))
 (segment (start 213.552401 79.969999) (end 212.929999 79.969999) (width 1) (layer F.Cu) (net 22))
 (segment (start 212.929999 79.969999) (end 212.09 80.809998) (width 1) (layer F.Cu) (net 22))
 (segment (start 212.09 80.809998) (end 212.09 82.17) (width 1) (layer F.Cu) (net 22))
 (segment (start 213.36 77.47) (end 210.09 80.74) (width 1) (layer F.Cu) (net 23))
 (segment (start 210.09 80.74) (end 210.09 82.17) (width 1) (layer F.Cu) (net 23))
 (segment (start 210.82 77.47) (end 208.09 80.2) (width 1) (layer F.Cu) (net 24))
 (segment (start 208.09 80.2) (end 208.09 82.17) (width 1) (layer F.Cu) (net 24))
 (segment (start 208.28 77.47) (end 206.09 79.66) (width 1) (layer F.Cu) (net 25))
 (segment (start 206.09 79.66) (end 206.09 82.17) (width 1) (layer F.Cu) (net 25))
 (segment (start 194.31 96.36) (end 194.56 96.36) (width 1) (layer F.Cu) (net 26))
 (segment (start 194.56 96.36) (end 196.11 94.81) (width 1) (layer F.Cu) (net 26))
 (segment (start 196.11 94.81) (end 209.23 94.81) (width 1) (layer F.Cu) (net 26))
 (segment (start 209.23 94.81) (end 210.09 95.67) (width 1) (layer F.Cu) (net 26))
 (segment (start 210.09 95.67) (end 210.09 98.17) (width 1) (layer F.Cu) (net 26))
 (segment (start 212.09 101.6) (end 212.09 98.17) (width 1) (layer F.Cu) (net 27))
 (segment (start 213.36 102.87) (end 212.09 101.6) (width 1) (layer F.Cu) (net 27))
 (segment (start 215.9 102.87) (end 214.09 101.06) (width 1) (layer F.Cu) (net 28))
 (segment (start 214.09 101.06) (end 214.09 98.17) (width 1) (layer F.Cu) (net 28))
 (segment (start 220.303619 78.394337) (end 219.71 78.987956) (width 0.4) (layer F.Cu) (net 29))
 (segment (start 217.35 100.33) (end 216.09 99.07) (width 0.4) (layer F.Cu) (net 29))
 (segment (start 218.018542 73.66) (end 219.71 75.351458) (width 0.4) (layer F.Cu) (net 29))
 (segment (start 194.31 73.66) (end 218.018542 73.66) (width 0.4) (layer F.Cu) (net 29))
 (segment (start 218.750002 100.33) (end 217.35 100.33) (width 0.4) (layer F.Cu) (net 29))
 (segment (start 220.30362 76.545664) (end 220.303619 78.394337) (width 0.4) (layer F.Cu) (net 29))
 (segment (start 216.09 99.07) (end 216.09 98.17) (width 0.4) (layer F.Cu) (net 29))
 (segment (start 192.63 80.955) (end 191.445 80.955) (width 0.4) (layer F.Cu) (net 29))
 (segment (start 191.445 80.955) (end 190.5 80.01) (width 0.4) (layer F.Cu) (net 29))
 (segment (start 219.71 99.370002) (end 218.750002 100.33) (width 0.4) (layer F.Cu) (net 29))
 (segment (start 190.5 80.01) (end 190.5 77.47) (width 0.4) (layer F.Cu) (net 29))
 (segment (start 190.5 77.47) (end 194.31 73.66) (width 0.4) (layer F.Cu) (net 29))
 (segment (start 219.71 75.351458) (end 219.71 75.952044) (width 0.4) (layer F.Cu) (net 29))
 (segment (start 219.71 75.952044) (end 220.30362 76.545664) (width 0.4) (layer F.Cu) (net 29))
 (segment (start 219.71 78.987956) (end 219.71 99.370002) (width 0.4) (layer F.Cu) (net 29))
 (segment (start 219.090001 78.759413) (end 219.09 96.27) (width 0.4) (layer F.Cu) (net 30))
 (segment (start 191.479999 77.760001) (end 194.31 74.93) (width 0.4) (layer F.Cu) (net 30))
 (segment (start 217.839414 74.93) (end 219.70361 76.794196) (width 0.4) (layer F.Cu) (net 30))
 (segment (start 219.70361 78.145804) (end 219.090001 78.759413) (width 0.4) (layer F.Cu) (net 30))
 (segment (start 218.09 97.27) (end 218.09 98.17) (width 0.4) (layer F.Cu) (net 30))
 (segment (start 191.479999 80.141457) (end 191.479999 77.760001) (width 0.4) (layer F.Cu) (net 30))
 (segment (start 194.31 74.93) (end 217.839414 74.93) (width 0.4) (layer F.Cu) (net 30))
 (segment (start 219.70361 76.794196) (end 219.70361 78.145804) (width 0.4) (layer F.Cu) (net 30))
 (segment (start 219.09 96.27) (end 218.09 97.27) (width 0.4) (layer F.Cu) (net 30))
 (segment (start 191.643541 80.304999) (end 191.479999 80.141457) (width 0.4) (layer F.Cu) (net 30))
 (segment (start 192.63 80.305) (end 191.643541 80.304999) (width 0.4) (layer F.Cu) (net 30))
 (segment (start 210.82 102.87) (end 210.82 102.270398) (width 1) (layer F.Cu) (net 31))
 (segment (start 208.09 99.540398) (end 208.09 98.17) (width 1) (layer F.Cu) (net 31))
 (segment (start 210.82 102.270398) (end 208.09 99.540398) (width 1) (layer F.Cu) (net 31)))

